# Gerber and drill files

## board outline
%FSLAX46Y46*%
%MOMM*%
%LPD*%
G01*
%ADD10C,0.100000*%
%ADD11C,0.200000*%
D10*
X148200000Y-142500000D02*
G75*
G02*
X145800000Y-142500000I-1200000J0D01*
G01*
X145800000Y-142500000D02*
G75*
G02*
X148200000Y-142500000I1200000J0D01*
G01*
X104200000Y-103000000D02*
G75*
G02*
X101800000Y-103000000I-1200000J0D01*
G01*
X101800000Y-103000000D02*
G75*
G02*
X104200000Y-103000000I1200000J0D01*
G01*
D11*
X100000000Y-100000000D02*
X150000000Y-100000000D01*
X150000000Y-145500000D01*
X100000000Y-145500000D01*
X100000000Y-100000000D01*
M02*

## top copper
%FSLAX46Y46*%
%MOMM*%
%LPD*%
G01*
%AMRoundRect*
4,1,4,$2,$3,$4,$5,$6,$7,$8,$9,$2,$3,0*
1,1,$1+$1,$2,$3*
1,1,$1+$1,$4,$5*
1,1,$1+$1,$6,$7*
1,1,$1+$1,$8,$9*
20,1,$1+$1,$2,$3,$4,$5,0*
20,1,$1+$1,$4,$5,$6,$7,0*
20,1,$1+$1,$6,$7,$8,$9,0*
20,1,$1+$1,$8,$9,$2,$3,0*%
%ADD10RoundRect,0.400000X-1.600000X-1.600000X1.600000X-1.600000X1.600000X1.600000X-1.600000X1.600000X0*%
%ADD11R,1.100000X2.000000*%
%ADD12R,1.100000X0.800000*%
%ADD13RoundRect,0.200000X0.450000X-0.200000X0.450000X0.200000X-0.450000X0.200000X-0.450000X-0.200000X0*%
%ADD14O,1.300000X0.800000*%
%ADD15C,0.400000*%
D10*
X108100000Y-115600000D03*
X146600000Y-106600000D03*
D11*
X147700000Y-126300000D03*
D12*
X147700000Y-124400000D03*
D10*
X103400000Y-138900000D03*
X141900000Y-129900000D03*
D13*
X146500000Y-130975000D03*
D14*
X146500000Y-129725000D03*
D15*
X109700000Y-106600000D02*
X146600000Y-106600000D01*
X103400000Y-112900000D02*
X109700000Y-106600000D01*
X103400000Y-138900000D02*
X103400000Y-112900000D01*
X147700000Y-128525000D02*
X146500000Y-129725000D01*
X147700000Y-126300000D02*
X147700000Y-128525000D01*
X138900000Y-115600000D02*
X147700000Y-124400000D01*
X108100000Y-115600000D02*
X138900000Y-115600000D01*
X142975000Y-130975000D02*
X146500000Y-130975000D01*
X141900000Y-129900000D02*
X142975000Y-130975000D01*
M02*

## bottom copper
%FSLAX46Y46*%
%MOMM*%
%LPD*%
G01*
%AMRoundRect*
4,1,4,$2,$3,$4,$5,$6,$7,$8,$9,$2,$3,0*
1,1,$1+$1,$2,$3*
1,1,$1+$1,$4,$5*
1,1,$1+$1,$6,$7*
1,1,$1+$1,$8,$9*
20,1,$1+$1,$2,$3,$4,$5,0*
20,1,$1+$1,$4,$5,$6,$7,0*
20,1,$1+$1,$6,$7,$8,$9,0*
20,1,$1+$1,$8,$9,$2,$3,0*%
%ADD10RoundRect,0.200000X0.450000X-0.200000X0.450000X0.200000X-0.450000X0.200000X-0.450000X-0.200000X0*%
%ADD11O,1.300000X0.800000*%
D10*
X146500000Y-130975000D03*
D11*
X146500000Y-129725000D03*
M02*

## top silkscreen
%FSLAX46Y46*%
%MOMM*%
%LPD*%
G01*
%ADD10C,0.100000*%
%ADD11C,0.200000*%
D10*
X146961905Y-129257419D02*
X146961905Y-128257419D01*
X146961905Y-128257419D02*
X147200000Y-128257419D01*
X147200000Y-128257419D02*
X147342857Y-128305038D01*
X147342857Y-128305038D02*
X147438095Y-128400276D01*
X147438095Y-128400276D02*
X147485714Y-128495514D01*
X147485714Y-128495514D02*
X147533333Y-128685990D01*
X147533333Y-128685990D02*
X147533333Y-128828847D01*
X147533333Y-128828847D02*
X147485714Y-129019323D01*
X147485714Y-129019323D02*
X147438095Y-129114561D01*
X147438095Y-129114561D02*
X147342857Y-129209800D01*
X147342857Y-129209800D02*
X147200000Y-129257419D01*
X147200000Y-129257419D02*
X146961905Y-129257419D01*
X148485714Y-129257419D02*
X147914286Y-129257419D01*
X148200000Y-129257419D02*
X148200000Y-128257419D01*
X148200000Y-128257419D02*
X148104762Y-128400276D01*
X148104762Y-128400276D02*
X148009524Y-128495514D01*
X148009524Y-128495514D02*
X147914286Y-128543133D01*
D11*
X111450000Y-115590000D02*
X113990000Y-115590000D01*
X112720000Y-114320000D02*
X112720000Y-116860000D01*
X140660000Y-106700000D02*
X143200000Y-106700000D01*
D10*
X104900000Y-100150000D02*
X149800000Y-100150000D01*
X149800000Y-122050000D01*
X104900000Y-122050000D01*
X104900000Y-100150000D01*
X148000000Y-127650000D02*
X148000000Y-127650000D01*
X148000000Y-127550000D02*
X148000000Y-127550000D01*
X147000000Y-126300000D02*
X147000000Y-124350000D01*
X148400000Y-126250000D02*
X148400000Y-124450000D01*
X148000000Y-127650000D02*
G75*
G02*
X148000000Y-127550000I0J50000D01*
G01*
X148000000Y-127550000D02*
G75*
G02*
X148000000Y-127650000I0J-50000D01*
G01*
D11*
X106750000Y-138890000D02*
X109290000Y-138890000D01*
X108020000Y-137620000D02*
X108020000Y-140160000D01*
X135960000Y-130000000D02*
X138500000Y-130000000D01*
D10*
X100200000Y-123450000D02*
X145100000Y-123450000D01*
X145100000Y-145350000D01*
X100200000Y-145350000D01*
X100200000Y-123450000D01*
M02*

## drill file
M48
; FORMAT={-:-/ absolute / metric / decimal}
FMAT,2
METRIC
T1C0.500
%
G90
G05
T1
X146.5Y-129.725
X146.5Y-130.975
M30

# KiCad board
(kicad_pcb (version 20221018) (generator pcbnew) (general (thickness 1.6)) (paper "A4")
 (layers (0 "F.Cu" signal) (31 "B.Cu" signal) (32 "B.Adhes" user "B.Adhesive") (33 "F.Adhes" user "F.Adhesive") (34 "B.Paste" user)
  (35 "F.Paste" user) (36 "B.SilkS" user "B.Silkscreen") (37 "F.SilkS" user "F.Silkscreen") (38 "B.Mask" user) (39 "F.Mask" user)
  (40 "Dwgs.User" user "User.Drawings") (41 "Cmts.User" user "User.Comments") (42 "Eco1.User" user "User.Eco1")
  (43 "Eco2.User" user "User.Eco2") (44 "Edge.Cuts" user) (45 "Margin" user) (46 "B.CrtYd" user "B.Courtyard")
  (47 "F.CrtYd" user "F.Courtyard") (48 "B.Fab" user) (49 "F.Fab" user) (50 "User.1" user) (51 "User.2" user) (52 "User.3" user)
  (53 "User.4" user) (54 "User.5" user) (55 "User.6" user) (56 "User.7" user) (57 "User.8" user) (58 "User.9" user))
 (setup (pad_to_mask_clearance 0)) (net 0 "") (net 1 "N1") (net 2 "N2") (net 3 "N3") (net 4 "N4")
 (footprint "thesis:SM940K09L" (layer "F.Cu") (at 105.1 100.35)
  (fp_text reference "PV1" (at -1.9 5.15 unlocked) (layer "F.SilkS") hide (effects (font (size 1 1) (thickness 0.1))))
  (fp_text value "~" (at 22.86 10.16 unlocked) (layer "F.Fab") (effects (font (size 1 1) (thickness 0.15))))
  (fp_line (start 6.35 15.24) (end 8.89 15.24) (stroke (width 0.2) (type default)) (layer "F.SilkS"))
  (fp_line (start 7.62 13.97) (end 7.62 16.51) (stroke (width 0.2) (type default)) (layer "F.SilkS"))
  (fp_line (start 35.56 6.35) (end 38.1 6.35) (stroke (width 0.2) (type default)) (layer "F.SilkS"))
  (fp_rect (start -0.2 -0.2) (end 44.7 21.7) (stroke (width 0.1) (type default)) (fill none) (layer "F.SilkS"))
  (pad "1" smd roundrect (at 3 15.25) (size 4 4) (layers "F.Cu" "F.Paste" "F.Mask") (roundrect_rratio 0.1) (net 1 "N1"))
  (pad "2" smd roundrect (at 41.5 6.25) (size 4 4) (layers "F.Cu" "F.Paste" "F.Mask") (roundrect_rratio 0.1) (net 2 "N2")))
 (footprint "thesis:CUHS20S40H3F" (layer "F.Cu") (at 147.7 125.35 90)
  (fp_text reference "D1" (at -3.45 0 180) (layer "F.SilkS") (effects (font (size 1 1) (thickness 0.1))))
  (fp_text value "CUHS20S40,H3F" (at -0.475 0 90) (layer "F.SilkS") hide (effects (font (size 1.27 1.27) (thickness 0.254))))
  (fp_line (start -2.3 0.3) (end -2.3 0.3) (stroke (width 0.1) (type solid)) (layer "F.SilkS"))
  (fp_line (start -2.2 0.3) (end -2.2 0.3) (stroke (width 0.1) (type solid)) (layer "F.SilkS"))
  (fp_line (start -0.95 -0.7) (end 1 -0.7) (stroke (width 0.1) (type solid)) (layer "F.SilkS"))
  (fp_line (start -0.9 0.7) (end 0.9 0.7) (stroke (width 0.1) (type solid)) (layer "F.SilkS"))
  (fp_arc (start -2.3 0.3) (mid -2.25 0.25) (end -2.2 0.3) (stroke (width 0.1) (type solid)) (layer "F.SilkS"))
  (fp_arc (start -2.2 0.3) (mid -2.25 0.35) (end -2.3 0.3) (stroke (width 0.1) (type solid)) (layer "F.SilkS"))
  (pad "1" smd rect (at -0.95 0 180) (size 1.1 2) (layers "F.Cu" "F.Paste" "F.Mask") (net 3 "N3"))
  (pad "2" smd rect (at 0.95 0 90) (size 0.8 1.1) (layers "F.Cu" "F.Paste" "F.Mask") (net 1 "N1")))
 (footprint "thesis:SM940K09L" (layer "F.Cu") (at 100.4 123.65)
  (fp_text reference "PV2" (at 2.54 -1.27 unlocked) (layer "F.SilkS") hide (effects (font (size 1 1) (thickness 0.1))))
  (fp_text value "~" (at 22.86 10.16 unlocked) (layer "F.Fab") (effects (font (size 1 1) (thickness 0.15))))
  (fp_line (start 6.35 15.24) (end 8.89 15.24) (stroke (width 0.2) (type default)) (layer "F.SilkS"))
  (fp_line (start 7.62 13.97) (end 7.62 16.51) (stroke (width 0.2) (type default)) (layer "F.SilkS"))
  (fp_line (start 35.56 6.35) (end 38.1 6.35) (stroke (width 0.2) (type default)) (layer "F.SilkS"))
  (fp_rect (start -0.2 -0.2) (end 44.7 21.7) (stroke (width 0.1) (type default)) (fill none) (layer "F.SilkS"))
  (pad "1" smd roundrect (at 3 15.25) (size 4 4) (layers "F.Cu" "F.Paste" "F.Mask") (roundrect_rratio 0.1) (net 2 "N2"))
  (pad "2" smd roundrect (at 41.5 6.25) (size 4 4) (layers "F.Cu" "F.Paste" "F.Mask") (roundrect_rratio 0.1) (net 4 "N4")))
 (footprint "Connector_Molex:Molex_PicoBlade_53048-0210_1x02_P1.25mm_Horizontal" (layer "B.Cu") (at 146.5 130.975 90)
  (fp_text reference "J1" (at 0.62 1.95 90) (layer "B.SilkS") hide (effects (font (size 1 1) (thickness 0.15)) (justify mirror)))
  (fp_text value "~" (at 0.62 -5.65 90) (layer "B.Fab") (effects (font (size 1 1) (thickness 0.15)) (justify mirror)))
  (pad "1" thru_hole roundrect (at 0 0 90) (size 0.8 1.3) (drill 0.5) (layers "*.Cu" "*.Mask") (roundrect_rratio 0.25) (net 4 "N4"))
  (pad "2" thru_hole oval (at 1.25 0 90) (size 0.8 1.3) (drill 0.5) (layers "*.Cu" "*.Mask") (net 3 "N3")))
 (gr_circle (center 147 142.5) (end 148.2 142.5) (stroke (width 0.1) (type default)) (fill none) (layer "Edge.Cuts"))
 (gr_circle (center 103 103) (end 104.2 103) (stroke (width 0.1) (type default)) (fill none) (layer "Edge.Cuts"))
 (gr_rect (start 100 100) (end 150 145.5) (stroke (width 0.2) (type default)) (fill none) (layer "Edge.Cuts"))
 (segment (start 109.7 106.6) (end 146.6 106.6) (width 0.4) (layer "F.Cu") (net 2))
 (segment (start 103.4 112.9) (end 109.7 106.6) (width 0.4) (layer "F.Cu") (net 2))
 (segment (start 103.4 138.9) (end 103.4 112.9) (width 0.4) (layer "F.Cu") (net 2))
 (segment (start 147.7 128.525) (end 146.5 129.725) (width 0.4) (layer "F.Cu") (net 3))
 (segment (start 147.7 126.3) (end 147.7 128.525) (width 0.4) (layer "F.Cu") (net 3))
 (segment (start 138.9 115.6) (end 147.7 124.4) (width 0.4) (layer "F.Cu") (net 1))
 (segment (start 108.1 115.6) (end 138.9 115.6) (width 0.4) (layer "F.Cu") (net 1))
 (segment (start 142.975 130.975) (end 146.5 130.975) (width 0.4) (layer "F.Cu") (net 4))
 (segment (start 141.9 129.9) (end 142.975 130.975) (width 0.4) (layer "F.Cu") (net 4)))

